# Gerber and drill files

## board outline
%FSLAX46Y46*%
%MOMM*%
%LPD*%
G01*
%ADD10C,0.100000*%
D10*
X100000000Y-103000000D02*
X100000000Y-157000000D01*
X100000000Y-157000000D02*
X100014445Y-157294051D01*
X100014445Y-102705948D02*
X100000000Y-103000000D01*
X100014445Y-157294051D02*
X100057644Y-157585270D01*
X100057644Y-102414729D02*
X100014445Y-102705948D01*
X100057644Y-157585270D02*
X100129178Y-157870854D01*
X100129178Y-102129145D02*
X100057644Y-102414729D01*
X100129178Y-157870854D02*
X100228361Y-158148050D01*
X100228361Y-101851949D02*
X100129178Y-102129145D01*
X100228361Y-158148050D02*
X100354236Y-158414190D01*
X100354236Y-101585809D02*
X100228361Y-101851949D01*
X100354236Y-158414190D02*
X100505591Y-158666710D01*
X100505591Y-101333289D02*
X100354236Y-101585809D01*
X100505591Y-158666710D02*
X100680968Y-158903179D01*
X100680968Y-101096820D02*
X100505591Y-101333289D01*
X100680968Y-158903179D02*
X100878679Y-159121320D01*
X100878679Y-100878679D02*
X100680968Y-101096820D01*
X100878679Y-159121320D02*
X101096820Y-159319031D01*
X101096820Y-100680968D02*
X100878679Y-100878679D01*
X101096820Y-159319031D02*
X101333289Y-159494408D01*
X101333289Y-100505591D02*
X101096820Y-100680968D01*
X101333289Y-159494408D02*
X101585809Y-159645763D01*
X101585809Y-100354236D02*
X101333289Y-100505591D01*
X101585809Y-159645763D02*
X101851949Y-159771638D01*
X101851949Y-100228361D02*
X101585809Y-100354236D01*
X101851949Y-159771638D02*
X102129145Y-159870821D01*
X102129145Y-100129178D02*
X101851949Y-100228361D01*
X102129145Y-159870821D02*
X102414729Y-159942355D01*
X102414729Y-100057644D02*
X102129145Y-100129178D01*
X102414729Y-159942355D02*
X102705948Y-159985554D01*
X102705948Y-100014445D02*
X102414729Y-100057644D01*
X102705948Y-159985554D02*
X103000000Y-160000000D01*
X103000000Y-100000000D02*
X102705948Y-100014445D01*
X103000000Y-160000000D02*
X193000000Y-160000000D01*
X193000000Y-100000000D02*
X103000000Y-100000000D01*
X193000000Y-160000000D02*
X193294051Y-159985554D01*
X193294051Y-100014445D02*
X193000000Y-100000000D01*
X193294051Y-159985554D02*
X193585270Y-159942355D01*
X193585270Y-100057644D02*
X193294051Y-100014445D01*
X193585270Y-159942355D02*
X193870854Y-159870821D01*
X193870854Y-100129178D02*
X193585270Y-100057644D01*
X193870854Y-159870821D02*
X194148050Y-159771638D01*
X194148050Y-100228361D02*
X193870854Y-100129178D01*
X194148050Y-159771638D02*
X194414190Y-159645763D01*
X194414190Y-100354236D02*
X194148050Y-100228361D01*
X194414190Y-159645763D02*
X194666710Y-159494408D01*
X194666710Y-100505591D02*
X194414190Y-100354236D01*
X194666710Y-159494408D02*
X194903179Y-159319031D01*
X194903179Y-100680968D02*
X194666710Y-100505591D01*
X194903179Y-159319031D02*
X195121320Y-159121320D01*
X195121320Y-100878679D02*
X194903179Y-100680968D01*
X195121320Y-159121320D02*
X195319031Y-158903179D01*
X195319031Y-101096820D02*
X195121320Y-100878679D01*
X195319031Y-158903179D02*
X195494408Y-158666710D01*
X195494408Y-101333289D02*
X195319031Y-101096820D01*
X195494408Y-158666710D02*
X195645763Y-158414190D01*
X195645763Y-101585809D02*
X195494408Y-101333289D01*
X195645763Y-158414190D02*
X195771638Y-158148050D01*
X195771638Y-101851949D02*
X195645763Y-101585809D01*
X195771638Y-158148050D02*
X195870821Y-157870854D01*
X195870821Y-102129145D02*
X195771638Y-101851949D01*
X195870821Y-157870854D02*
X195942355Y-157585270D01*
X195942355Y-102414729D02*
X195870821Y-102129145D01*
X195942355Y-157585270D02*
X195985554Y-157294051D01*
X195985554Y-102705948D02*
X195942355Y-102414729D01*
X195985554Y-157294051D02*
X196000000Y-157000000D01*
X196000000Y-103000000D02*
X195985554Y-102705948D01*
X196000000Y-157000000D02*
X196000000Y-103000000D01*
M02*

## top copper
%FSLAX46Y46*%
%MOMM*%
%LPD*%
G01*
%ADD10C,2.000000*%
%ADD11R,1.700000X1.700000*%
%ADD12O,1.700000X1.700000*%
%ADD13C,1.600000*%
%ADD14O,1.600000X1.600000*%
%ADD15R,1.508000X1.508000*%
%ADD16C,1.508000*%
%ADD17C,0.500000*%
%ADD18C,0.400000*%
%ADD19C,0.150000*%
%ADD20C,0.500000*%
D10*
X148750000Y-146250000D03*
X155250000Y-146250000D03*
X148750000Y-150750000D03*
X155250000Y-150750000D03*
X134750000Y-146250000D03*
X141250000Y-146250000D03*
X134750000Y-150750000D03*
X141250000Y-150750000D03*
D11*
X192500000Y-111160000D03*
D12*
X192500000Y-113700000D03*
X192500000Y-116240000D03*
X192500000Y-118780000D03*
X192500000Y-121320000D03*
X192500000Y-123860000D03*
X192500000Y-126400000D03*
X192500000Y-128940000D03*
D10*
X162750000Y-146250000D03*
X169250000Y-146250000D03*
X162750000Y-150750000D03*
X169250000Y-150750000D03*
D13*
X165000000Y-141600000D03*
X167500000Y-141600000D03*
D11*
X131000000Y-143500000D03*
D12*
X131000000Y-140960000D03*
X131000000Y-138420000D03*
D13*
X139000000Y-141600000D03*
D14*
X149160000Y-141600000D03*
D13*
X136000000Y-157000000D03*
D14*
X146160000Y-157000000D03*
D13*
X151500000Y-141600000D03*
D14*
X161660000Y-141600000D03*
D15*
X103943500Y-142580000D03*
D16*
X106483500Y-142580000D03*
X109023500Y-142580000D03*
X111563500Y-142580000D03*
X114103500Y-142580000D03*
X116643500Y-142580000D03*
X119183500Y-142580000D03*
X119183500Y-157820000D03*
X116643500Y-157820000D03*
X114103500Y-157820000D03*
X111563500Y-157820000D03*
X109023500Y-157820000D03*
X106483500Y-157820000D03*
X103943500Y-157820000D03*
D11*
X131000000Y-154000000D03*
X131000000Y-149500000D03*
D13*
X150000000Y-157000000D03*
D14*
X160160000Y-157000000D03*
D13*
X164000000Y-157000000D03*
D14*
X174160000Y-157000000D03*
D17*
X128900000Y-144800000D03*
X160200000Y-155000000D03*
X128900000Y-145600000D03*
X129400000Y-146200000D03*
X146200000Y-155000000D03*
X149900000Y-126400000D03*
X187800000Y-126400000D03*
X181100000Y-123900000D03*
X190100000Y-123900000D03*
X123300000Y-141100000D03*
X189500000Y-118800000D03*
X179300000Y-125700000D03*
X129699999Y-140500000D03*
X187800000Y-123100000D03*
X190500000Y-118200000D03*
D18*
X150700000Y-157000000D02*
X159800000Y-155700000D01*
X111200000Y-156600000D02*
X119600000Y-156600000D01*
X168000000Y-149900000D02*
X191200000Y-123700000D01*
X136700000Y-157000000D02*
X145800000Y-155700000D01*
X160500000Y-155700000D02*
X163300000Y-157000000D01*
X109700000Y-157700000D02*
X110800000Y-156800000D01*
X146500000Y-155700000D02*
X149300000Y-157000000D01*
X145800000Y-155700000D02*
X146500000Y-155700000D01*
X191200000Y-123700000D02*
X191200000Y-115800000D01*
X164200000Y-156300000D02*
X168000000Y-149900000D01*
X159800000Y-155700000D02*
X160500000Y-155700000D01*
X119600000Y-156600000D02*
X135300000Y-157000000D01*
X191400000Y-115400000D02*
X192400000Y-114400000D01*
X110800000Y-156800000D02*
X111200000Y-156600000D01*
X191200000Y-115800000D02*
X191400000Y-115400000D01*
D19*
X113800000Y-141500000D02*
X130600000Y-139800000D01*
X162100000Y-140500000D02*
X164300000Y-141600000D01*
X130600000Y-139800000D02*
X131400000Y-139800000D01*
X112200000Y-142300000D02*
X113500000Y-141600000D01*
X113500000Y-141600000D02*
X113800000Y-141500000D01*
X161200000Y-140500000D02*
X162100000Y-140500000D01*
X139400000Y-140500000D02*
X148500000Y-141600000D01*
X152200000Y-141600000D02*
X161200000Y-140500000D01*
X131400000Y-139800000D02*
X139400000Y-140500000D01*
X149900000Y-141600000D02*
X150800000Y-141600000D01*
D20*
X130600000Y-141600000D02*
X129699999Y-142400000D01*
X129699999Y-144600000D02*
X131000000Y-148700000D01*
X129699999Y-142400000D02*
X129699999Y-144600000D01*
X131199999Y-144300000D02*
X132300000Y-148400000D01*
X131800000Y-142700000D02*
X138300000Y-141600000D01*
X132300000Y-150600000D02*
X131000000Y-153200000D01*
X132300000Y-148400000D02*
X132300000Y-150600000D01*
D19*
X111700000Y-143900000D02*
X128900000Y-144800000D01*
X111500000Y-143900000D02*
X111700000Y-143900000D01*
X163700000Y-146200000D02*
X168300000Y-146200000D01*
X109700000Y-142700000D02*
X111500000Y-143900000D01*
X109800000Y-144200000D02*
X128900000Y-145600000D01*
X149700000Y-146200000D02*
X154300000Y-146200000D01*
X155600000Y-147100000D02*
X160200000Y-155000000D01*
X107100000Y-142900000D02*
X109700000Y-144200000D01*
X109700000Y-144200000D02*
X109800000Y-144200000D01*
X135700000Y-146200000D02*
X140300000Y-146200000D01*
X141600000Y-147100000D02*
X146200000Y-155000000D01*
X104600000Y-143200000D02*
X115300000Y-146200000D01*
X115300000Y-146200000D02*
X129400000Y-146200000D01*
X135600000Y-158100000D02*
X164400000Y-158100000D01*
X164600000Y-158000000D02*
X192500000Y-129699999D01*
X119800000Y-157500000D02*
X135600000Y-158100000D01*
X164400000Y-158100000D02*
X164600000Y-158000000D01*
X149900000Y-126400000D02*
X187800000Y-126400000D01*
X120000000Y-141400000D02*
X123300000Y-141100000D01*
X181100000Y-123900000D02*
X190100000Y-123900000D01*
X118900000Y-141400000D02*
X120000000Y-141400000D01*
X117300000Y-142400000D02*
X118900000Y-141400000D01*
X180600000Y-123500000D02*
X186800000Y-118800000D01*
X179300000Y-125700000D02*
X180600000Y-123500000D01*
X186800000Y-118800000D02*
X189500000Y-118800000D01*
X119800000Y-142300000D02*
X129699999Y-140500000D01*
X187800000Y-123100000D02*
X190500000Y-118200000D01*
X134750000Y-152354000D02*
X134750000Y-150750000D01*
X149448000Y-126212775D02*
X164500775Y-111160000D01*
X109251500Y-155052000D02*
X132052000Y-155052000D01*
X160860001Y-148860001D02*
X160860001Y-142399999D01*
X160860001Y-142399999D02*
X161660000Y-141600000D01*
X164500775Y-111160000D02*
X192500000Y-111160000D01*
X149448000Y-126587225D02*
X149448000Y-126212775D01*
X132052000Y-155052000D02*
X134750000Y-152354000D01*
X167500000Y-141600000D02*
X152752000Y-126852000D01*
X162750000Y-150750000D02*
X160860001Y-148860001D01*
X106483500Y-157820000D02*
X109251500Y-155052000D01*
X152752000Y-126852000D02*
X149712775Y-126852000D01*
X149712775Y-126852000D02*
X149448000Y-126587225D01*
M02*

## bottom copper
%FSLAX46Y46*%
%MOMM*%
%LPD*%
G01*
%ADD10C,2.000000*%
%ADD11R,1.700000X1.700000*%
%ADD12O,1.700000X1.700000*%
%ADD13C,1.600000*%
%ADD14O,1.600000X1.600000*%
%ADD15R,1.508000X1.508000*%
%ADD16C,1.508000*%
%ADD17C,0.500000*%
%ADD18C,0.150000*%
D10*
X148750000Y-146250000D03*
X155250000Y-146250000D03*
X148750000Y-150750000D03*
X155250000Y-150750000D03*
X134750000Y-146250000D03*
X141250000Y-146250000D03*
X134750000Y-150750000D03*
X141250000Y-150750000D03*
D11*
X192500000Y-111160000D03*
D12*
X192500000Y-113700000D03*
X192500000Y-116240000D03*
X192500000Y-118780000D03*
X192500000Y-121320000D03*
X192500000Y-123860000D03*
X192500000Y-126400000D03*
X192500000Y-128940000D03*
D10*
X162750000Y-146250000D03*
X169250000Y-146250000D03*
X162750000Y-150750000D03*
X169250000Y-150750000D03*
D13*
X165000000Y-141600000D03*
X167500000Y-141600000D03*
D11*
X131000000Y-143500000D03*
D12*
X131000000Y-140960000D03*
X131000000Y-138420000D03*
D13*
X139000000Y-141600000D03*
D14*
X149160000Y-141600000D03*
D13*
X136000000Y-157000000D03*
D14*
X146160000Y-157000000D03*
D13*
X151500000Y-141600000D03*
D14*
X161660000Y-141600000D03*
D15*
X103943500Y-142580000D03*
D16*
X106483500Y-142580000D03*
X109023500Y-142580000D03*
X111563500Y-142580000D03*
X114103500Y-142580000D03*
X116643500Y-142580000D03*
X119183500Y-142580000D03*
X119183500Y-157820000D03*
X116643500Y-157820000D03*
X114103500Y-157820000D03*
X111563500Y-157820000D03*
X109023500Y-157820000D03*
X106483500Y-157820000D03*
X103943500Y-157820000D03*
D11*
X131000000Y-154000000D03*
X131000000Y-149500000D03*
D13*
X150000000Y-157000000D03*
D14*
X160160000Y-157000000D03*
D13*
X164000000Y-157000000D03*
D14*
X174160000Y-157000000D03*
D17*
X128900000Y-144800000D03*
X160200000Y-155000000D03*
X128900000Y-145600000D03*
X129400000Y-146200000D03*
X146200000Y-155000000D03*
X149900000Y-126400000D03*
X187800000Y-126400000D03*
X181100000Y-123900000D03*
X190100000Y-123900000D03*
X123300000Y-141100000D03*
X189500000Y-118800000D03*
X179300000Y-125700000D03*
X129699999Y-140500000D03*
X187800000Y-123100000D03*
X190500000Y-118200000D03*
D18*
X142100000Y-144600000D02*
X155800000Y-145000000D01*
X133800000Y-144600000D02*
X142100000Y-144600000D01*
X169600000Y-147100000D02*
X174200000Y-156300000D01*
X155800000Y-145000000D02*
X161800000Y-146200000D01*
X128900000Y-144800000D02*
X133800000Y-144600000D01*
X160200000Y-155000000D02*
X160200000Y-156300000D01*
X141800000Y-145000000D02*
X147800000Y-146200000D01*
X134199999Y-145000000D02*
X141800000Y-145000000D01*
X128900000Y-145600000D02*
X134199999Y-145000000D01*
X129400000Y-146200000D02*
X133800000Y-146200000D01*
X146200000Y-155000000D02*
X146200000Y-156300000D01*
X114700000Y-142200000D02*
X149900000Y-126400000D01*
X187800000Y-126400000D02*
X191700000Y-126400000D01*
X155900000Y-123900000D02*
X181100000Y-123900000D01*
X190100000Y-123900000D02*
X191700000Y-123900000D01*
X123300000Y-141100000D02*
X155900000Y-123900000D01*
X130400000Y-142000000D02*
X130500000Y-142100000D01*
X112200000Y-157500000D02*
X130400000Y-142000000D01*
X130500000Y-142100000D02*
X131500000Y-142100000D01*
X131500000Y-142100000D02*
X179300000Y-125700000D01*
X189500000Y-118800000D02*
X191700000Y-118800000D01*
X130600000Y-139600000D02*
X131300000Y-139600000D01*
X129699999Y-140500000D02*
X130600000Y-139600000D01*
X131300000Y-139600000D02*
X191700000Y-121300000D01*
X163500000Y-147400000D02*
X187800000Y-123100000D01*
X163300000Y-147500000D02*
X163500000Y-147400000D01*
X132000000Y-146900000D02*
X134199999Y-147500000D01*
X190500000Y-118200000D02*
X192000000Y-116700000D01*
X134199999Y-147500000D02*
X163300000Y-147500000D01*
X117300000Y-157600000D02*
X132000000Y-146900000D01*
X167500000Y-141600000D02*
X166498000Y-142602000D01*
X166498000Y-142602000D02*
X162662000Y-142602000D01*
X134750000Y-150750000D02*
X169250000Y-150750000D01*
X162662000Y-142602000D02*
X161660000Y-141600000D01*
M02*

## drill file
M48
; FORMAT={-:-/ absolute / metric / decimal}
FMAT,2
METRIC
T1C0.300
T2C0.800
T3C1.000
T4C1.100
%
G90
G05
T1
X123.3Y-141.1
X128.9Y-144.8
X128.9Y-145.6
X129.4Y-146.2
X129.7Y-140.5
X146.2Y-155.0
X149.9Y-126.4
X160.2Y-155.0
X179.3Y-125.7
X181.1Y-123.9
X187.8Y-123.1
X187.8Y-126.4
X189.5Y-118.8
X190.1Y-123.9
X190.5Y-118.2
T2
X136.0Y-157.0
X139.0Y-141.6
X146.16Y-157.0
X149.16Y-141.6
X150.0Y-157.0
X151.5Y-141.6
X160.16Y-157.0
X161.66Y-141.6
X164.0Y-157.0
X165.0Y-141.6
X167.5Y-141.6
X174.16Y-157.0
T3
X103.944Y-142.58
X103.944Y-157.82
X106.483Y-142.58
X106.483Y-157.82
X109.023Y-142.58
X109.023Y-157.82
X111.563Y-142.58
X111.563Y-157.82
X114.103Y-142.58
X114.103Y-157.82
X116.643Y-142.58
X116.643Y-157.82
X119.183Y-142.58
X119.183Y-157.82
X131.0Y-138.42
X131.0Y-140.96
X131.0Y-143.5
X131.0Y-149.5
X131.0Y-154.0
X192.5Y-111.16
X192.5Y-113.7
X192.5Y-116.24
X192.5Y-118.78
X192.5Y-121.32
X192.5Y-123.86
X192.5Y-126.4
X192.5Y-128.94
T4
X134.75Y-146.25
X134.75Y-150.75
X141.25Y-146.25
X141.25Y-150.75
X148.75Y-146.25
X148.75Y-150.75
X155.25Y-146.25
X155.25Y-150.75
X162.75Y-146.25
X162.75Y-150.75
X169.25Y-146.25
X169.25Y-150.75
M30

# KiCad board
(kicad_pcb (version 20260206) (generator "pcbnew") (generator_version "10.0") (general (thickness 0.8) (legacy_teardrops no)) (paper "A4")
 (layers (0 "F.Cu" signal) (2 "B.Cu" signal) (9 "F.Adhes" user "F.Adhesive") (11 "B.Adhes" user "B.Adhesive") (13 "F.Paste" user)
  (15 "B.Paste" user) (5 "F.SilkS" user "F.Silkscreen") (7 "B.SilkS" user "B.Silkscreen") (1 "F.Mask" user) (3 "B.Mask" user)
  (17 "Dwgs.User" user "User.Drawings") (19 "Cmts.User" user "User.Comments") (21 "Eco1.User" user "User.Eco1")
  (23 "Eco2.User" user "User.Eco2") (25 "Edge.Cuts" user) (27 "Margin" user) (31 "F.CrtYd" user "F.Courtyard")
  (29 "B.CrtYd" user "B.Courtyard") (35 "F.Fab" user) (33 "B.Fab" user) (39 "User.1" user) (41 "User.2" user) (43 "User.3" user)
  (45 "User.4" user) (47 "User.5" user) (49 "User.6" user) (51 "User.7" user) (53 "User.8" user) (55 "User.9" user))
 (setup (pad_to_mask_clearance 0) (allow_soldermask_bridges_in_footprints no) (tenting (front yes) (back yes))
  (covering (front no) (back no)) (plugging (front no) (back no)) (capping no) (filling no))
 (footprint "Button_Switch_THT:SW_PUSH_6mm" (layer "F.Cu") (at 148.75 146.25)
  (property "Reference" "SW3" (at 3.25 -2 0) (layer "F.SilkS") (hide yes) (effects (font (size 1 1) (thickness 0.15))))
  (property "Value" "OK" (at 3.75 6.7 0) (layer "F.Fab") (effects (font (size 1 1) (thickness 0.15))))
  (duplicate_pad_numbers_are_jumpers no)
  (pad "1" thru_hole circle (at 0 0 90) (size 2 2) (drill 1.1) (layers "*.Cu" "*.Mask") (remove_unused_layers no) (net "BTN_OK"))
  (pad "1" thru_hole circle (at 6.5 0 90) (size 2 2) (drill 1.1) (layers "*.Cu" "*.Mask") (remove_unused_layers no) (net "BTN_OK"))
  (pad "2" thru_hole circle (at 0 4.5 90) (size 2 2) (drill 1.1) (layers "*.Cu" "*.Mask") (remove_unused_layers no) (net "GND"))
  (pad "2" thru_hole circle (at 6.5 4.5 90) (size 2 2) (drill 1.1) (layers "*.Cu" "*.Mask") (remove_unused_layers no) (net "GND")))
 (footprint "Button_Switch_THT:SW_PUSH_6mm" (layer "F.Cu") (at 134.75 146.25)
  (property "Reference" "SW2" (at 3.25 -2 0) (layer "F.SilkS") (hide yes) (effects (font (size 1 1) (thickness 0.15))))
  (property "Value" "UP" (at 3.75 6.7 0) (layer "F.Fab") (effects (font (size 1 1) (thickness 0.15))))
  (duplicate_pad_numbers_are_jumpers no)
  (pad "1" thru_hole circle (at 0 0 90) (size 2 2) (drill 1.1) (layers "*.Cu" "*.Mask") (remove_unused_layers no) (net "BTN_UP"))
  (pad "1" thru_hole circle (at 6.5 0 90) (size 2 2) (drill 1.1) (layers "*.Cu" "*.Mask") (remove_unused_layers no) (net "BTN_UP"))
  (pad "2" thru_hole circle (at 0 4.5 90) (size 2 2) (drill 1.1) (layers "*.Cu" "*.Mask") (remove_unused_layers no) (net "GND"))
  (pad "2" thru_hole circle (at 6.5 4.5 90) (size 2 2) (drill 1.1) (layers "*.Cu" "*.Mask") (remove_unused_layers no) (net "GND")))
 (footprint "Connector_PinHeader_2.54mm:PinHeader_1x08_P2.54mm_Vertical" (layer "F.Cu") (at 192.5 111.16)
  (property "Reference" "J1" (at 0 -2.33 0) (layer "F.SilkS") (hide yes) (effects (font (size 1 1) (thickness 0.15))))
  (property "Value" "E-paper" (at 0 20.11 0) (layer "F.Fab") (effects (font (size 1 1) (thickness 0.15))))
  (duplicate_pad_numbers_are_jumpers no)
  (pad "1" thru_hole rect (at 0 0) (size 1.7 1.7) (drill 1) (layers "*.Cu" "*.Mask") (remove_unused_layers no) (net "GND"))
  (pad "2" thru_hole oval (at 0 2.54) (size 1.7 1.7) (drill 1) (layers "*.Cu" "*.Mask") (remove_unused_layers no) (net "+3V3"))
  (pad "3" thru_hole oval (at 0 5.08) (size 1.7 1.7) (drill 1) (layers "*.Cu" "*.Mask") (remove_unused_layers no) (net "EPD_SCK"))
  (pad "4" thru_hole oval (at 0 7.62) (size 1.7 1.7) (drill 1) (layers "*.Cu" "*.Mask") (remove_unused_layers no) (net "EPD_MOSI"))
  (pad "5" thru_hole oval (at 0 10.16) (size 1.7 1.7) (drill 1) (layers "*.Cu" "*.Mask") (remove_unused_layers no) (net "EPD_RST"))
  (pad "6" thru_hole oval (at 0 12.7) (size 1.7 1.7) (drill 1) (layers "*.Cu" "*.Mask") (remove_unused_layers no) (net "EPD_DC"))
  (pad "7" thru_hole oval (at 0 15.24) (size 1.7 1.7) (drill 1) (layers "*.Cu" "*.Mask") (remove_unused_layers no) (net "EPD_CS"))
  (pad "8" thru_hole oval (at 0 17.78) (size 1.7 1.7) (drill 1) (layers "*.Cu" "*.Mask") (remove_unused_layers no) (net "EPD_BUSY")))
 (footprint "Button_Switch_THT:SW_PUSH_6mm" (layer "F.Cu") (at 162.75 146.25)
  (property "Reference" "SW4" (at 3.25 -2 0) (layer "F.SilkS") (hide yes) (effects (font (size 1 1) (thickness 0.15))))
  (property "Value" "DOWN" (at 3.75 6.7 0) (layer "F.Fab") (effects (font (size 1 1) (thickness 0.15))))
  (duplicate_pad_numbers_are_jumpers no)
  (pad "1" thru_hole circle (at 0 0 90) (size 2 2) (drill 1.1) (layers "*.Cu" "*.Mask") (remove_unused_layers no) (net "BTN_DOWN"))
  (pad "1" thru_hole circle (at 6.5 0 90) (size 2 2) (drill 1.1) (layers "*.Cu" "*.Mask") (remove_unused_layers no) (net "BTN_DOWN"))
  (pad "2" thru_hole circle (at 0 4.5 90) (size 2 2) (drill 1.1) (layers "*.Cu" "*.Mask") (remove_unused_layers no) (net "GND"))
  (pad "2" thru_hole circle (at 6.5 4.5 90) (size 2 2) (drill 1.1) (layers "*.Cu" "*.Mask") (remove_unused_layers no) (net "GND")))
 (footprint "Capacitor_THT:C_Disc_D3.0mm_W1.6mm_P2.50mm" (layer "B.Cu") (at 165 141.6)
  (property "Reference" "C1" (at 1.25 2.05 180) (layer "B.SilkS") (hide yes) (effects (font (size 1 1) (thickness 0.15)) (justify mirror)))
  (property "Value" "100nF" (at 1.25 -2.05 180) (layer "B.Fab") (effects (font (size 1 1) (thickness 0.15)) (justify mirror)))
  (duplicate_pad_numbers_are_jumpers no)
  (pad "1" thru_hole circle (at 0 0) (size 1.6 1.6) (drill 0.8) (layers "*.Cu" "*.Mask") (remove_unused_layers no) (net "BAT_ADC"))
  (pad "2" thru_hole circle (at 2.5 0) (size 1.6 1.6) (drill 0.8) (layers "*.Cu" "*.Mask") (remove_unused_layers no) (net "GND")))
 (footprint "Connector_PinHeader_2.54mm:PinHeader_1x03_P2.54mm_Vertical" (layer "B.Cu") (at 131 143.5)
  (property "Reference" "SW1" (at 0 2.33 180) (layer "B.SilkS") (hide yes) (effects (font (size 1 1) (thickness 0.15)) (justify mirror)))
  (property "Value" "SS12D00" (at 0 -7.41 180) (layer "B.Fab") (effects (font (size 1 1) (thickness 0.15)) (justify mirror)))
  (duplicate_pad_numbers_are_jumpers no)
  (pad "1" thru_hole rect (at 0 0) (size 1.7 1.7) (drill 1) (layers "*.Cu" "*.Mask") (remove_unused_layers no) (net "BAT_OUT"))
  (pad "2" thru_hole oval (at 0 -2.54) (size 1.7 1.7) (drill 1) (layers "*.Cu" "*.Mask") (remove_unused_layers no) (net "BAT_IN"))
  (pad "3" thru_hole oval (at 0 -5.08) (size 1.7 1.7) (drill 1) (layers "*.Cu" "*.Mask") (remove_unused_layers no)))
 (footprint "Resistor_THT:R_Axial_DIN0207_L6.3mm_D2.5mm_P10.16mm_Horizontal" (layer "B.Cu") (at 139 141.6)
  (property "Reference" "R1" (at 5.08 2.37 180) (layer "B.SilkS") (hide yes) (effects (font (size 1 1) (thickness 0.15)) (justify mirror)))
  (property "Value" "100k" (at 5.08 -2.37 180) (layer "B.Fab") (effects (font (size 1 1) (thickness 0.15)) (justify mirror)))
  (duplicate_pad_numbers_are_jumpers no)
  (pad "1" thru_hole circle (at 0 0) (size 1.6 1.6) (drill 0.8) (layers "*.Cu" "*.Mask") (remove_unused_layers no) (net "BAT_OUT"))
  (pad "2" thru_hole oval (at 10.16 0) (size 1.6 1.6) (drill 0.8) (layers "*.Cu" "*.Mask") (remove_unused_layers no) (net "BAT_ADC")))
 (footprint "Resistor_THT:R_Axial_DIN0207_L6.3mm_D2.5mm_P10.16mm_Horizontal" (layer "B.Cu") (at 136 157)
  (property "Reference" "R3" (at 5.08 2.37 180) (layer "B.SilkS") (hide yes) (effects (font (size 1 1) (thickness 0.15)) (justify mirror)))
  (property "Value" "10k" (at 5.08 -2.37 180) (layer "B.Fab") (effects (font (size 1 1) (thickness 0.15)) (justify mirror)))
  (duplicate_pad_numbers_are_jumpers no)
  (pad "1" thru_hole circle (at 0 0) (size 1.6 1.6) (drill 0.8) (layers "*.Cu" "*.Mask") (remove_unused_layers no) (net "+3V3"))
  (pad "2" thru_hole oval (at 10.16 0) (size 1.6 1.6) (drill 0.8) (layers "*.Cu" "*.Mask") (remove_unused_layers no) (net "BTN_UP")))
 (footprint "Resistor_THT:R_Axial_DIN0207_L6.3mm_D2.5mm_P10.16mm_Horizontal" (layer "B.Cu") (at 151.5 141.6)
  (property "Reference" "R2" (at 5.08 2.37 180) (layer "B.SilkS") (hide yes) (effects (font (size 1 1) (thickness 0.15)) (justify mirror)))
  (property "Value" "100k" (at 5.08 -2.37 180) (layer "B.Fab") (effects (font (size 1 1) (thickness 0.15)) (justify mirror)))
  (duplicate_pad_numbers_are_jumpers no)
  (pad "1" thru_hole circle (at 0 0) (size 1.6 1.6) (drill 0.8) (layers "*.Cu" "*.Mask") (remove_unused_layers no) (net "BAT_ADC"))
  (pad "2" thru_hole oval (at 10.16 0) (size 1.6 1.6) (drill 0.8) (layers "*.Cu" "*.Mask") (remove_unused_layers no) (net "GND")))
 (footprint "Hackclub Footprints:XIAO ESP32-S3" (layer "B.Cu") (at 111.5 150.2 -90)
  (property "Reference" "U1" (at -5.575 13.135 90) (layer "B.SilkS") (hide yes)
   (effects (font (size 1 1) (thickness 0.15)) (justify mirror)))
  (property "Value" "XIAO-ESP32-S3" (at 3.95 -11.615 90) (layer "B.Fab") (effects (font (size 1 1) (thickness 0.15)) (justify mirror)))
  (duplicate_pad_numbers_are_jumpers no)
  (pad "1" thru_hole rect (at -7.62 7.5565 270) (size 1.508 1.508) (drill 1) (layers "*.Cu" "*.Mask") (remove_unused_layers no)
   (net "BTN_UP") (solder_mask_margin 0.102))
  (pad "2" thru_hole circle (at -7.62 5.0165 270) (size 1.508 1.508) (drill 1) (layers "*.Cu" "*.Mask") (remove_unused_layers no)
   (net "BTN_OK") (solder_mask_margin 0.102))
  (pad "3" thru_hole circle (at -7.62 2.4765 270) (size 1.508 1.508) (drill 1) (layers "*.Cu" "*.Mask") (remove_unused_layers no)
   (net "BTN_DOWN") (solder_mask_margin 0.102))
  (pad "4" thru_hole circle (at -7.62 -0.0635 270) (size 1.508 1.508) (drill 1) (layers "*.Cu" "*.Mask") (remove_unused_layers no)
   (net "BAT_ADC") (solder_mask_margin 0.102))
  (pad "5" thru_hole circle (at -7.62 -2.6035 270) (size 1.508 1.508) (drill 1) (layers "*.Cu" "*.Mask") (remove_unused_layers no)
   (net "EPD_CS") (solder_mask_margin 0.102))
  (pad "6" thru_hole circle (at -7.62 -5.1435 270) (size 1.508 1.508) (drill 1) (layers "*.Cu" "*.Mask") (remove_unused_layers no)
   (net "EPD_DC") (solder_mask_margin 0.102))
  (pad "7" thru_hole circle (at -7.62 -7.6835 270) (size 1.508 1.508) (drill 1) (layers "*.Cu" "*.Mask") (remove_unused_layers no)
   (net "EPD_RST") (solder_mask_margin 0.102))
  (pad "8" thru_hole circle (at 7.62 -7.6835 270) (size 1.508 1.508) (drill 1) (layers "*.Cu" "*.Mask") (remove_unused_layers no)
   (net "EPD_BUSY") (solder_mask_margin 0.102))
  (pad "9" thru_hole circle (at 7.62 -5.1435 270) (size 1.508 1.508) (drill 1) (layers "*.Cu" "*.Mask") (remove_unused_layers no)
   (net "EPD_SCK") (solder_mask_margin 0.102))
  (pad "10" thru_hole circle (at 7.62 -2.6035 270) (size 1.508 1.508) (drill 1) (layers "*.Cu" "*.Mask") (remove_unused_layers no)
   (solder_mask_margin 0.102))
  (pad "11" thru_hole circle (at 7.62 -0.0635 270) (size 1.508 1.508) (drill 1) (layers "*.Cu" "*.Mask") (remove_unused_layers no)
   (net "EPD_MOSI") (solder_mask_margin 0.102))
  (pad "12" thru_hole circle (at 7.62 2.4765 270) (size 1.508 1.508) (drill 1) (layers "*.Cu" "*.Mask") (remove_unused_layers no)
   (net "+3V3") (solder_mask_margin 0.102))
  (pad "13" thru_hole circle (at 7.62 5.0165 270) (size 1.508 1.508) (drill 1) (layers "*.Cu" "*.Mask") (remove_unused_layers no)
   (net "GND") (solder_mask_margin 0.102))
  (pad "14" thru_hole circle (at 7.62 7.5565 270) (size 1.508 1.508) (drill 1) (layers "*.Cu" "*.Mask") (remove_unused_layers no)
   (solder_mask_margin 0.102)))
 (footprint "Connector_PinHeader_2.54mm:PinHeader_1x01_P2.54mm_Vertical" (layer "B.Cu") (at 131 154)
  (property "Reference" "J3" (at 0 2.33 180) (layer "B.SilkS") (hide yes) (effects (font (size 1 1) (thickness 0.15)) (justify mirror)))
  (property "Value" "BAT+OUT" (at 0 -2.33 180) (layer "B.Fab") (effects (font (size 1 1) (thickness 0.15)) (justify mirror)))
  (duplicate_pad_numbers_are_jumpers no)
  (pad "1" thru_hole rect (at 0 0) (size 1.7 1.7) (drill 1) (layers "*.Cu" "*.Mask") (remove_unused_layers no) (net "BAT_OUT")))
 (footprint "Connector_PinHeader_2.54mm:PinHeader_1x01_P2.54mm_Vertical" (layer "B.Cu") (at 131 149.5)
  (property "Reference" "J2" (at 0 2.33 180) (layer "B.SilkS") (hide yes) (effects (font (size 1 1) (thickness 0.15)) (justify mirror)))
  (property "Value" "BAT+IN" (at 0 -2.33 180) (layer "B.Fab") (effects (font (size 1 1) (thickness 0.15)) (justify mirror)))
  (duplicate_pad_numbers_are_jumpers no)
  (pad "1" thru_hole rect (at 0 0) (size 1.7 1.7) (drill 1) (layers "*.Cu" "*.Mask") (remove_unused_layers no) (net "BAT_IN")))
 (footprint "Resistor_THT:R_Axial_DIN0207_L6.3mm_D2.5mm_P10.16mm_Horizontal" (layer "B.Cu") (at 150 157)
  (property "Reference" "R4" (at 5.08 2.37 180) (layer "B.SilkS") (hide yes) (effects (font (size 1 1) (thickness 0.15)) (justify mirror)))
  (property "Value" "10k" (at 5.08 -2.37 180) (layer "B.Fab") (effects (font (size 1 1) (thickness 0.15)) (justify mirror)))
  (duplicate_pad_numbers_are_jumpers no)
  (pad "1" thru_hole circle (at 0 0) (size 1.6 1.6) (drill 0.8) (layers "*.Cu" "*.Mask") (remove_unused_layers no) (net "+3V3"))
  (pad "2" thru_hole oval (at 10.16 0) (size 1.6 1.6) (drill 0.8) (layers "*.Cu" "*.Mask") (remove_unused_layers no) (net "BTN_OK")))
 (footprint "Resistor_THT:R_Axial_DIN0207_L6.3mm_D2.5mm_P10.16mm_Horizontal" (layer "B.Cu") (at 164 157)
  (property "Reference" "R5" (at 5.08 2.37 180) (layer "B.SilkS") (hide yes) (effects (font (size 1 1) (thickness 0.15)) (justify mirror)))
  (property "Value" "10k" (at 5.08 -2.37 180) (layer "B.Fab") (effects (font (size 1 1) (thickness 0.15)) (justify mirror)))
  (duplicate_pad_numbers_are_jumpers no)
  (pad "1" thru_hole circle (at 0 0) (size 1.6 1.6) (drill 0.8) (layers "*.Cu" "*.Mask") (remove_unused_layers no) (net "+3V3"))
  (pad "2" thru_hole oval (at 10.16 0) (size 1.6 1.6) (drill 0.8) (layers "*.Cu" "*.Mask") (remove_unused_layers no) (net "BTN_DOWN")))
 (gr_line (start 100 103) (end 100 157) (stroke (width 0.1) (type default)) (layer "Edge.Cuts"))
 (gr_line (start 100 157) (end 100.014445 157.294051) (stroke (width 0.1) (type default)) (layer "Edge.Cuts"))
 (gr_line (start 100.014445 102.705948) (end 100 103) (stroke (width 0.1) (type default)) (layer "Edge.Cuts"))
 (gr_line (start 100.014445 157.294051) (end 100.057644 157.58527) (stroke (width 0.1) (type default)) (layer "Edge.Cuts"))
 (gr_line (start 100.057644 102.414729) (end 100.014445 102.705948) (stroke (width 0.1) (type default)) (layer "Edge.Cuts"))
 (gr_line (start 100.057644 157.58527) (end 100.129178 157.870854) (stroke (width 0.1) (type default)) (layer "Edge.Cuts"))
 (gr_line (start 100.129178 102.129145) (end 100.057644 102.414729) (stroke (width 0.1) (type default)) (layer "Edge.Cuts"))
 (gr_line (start 100.129178 157.870854) (end 100.228361 158.14805) (stroke (width 0.1) (type default)) (layer "Edge.Cuts"))
 (gr_line (start 100.228361 101.851949) (end 100.129178 102.129145) (stroke (width 0.1) (type default)) (layer "Edge.Cuts"))
 (gr_line (start 100.228361 158.14805) (end 100.354236 158.41419) (stroke (width 0.1) (type default)) (layer "Edge.Cuts"))
 (gr_line (start 100.354236 101.585809) (end 100.228361 101.851949) (stroke (width 0.1) (type default)) (layer "Edge.Cuts"))
 (gr_line (start 100.354236 158.41419) (end 100.505591 158.66671) (stroke (width 0.1) (type default)) (layer "Edge.Cuts"))
 (gr_line (start 100.505591 101.333289) (end 100.354236 101.585809) (stroke (width 0.1) (type default)) (layer "Edge.Cuts"))
 (gr_line (start 100.505591 158.66671) (end 100.680968 158.903179) (stroke (width 0.1) (type default)) (layer "Edge.Cuts"))
 (gr_line (start 100.680968 101.09682) (end 100.505591 101.333289) (stroke (width 0.1) (type default)) (layer "Edge.Cuts"))
 (gr_line (start 100.680968 158.903179) (end 100.878679 159.12132) (stroke (width 0.1) (type default)) (layer "Edge.Cuts"))
 (gr_line (start 100.878679 100.878679) (end 100.680968 101.09682) (stroke (width 0.1) (type default)) (layer "Edge.Cuts"))
 (gr_line (start 100.878679 159.12132) (end 101.09682 159.319031) (stroke (width 0.1) (type default)) (layer "Edge.Cuts"))
 (gr_line (start 101.09682 100.680968) (end 100.878679 100.878679) (stroke (width 0.1) (type default)) (layer "Edge.Cuts"))
 (gr_line (start 101.09682 159.319031) (end 101.333289 159.494408) (stroke (width 0.1) (type default)) (layer "Edge.Cuts"))
 (gr_line (start 101.333289 100.505591) (end 101.09682 100.680968) (stroke (width 0.1) (type default)) (layer "Edge.Cuts"))
 (gr_line (start 101.333289 159.494408) (end 101.585809 159.645763) (stroke (width 0.1) (type default)) (layer "Edge.Cuts"))
 (gr_line (start 101.585809 100.354236) (end 101.333289 100.505591) (stroke (width 0.1) (type default)) (layer "Edge.Cuts"))
 (gr_line (start 101.585809 159.645763) (end 101.851949 159.771638) (stroke (width 0.1) (type default)) (layer "Edge.Cuts"))
 (gr_line (start 101.851949 100.228361) (end 101.585809 100.354236) (stroke (width 0.1) (type default)) (layer "Edge.Cuts"))
 (gr_line (start 101.851949 159.771638) (end 102.129145 159.870821) (stroke (width 0.1) (type default)) (layer "Edge.Cuts"))
 (gr_line (start 102.129145 100.129178) (end 101.851949 100.228361) (stroke (width 0.1) (type default)) (layer "Edge.Cuts"))
 (gr_line (start 102.129145 159.870821) (end 102.414729 159.942355) (stroke (width 0.1) (type default)) (layer "Edge.Cuts"))
 (gr_line (start 102.414729 100.057644) (end 102.129145 100.129178) (stroke (width 0.1) (type default)) (layer "Edge.Cuts"))
 (gr_line (start 102.414729 159.942355) (end 102.705948 159.985554) (stroke (width 0.1) (type default)) (layer "Edge.Cuts"))
 (gr_line (start 102.705948 100.014445) (end 102.414729 100.057644) (stroke (width 0.1) (type default)) (layer "Edge.Cuts"))
 (gr_line (start 102.705948 159.985554) (end 103 160) (stroke (width 0.1) (type default)) (layer "Edge.Cuts"))
 (gr_line (start 103 100) (end 102.705948 100.014445) (stroke (width 0.1) (type default)) (layer "Edge.Cuts"))
 (gr_line (start 103 160) (end 193 160) (stroke (width 0.1) (type default)) (layer "Edge.Cuts"))
 (gr_line (start 193 100) (end 103 100) (stroke (width 0.1) (type default)) (layer "Edge.Cuts"))
 (gr_line (start 193 160) (end 193.294051 159.985554) (stroke (width 0.1) (type default)) (layer "Edge.Cuts"))
 (gr_line (start 193.294051 100.014445) (end 193 100) (stroke (width 0.1) (type default)) (layer "Edge.Cuts"))
 (gr_line (start 193.294051 159.985554) (end 193.58527 159.942355) (stroke (width 0.1) (type default)) (layer "Edge.Cuts"))
 (gr_line (start 193.58527 100.057644) (end 193.294051 100.014445) (stroke (width 0.1) (type default)) (layer "Edge.Cuts"))
 (gr_line (start 193.58527 159.942355) (end 193.870854 159.870821) (stroke (width 0.1) (type default)) (layer "Edge.Cuts"))
 (gr_line (start 193.870854 100.129178) (end 193.58527 100.057644) (stroke (width 0.1) (type default)) (layer "Edge.Cuts"))
 (gr_line (start 193.870854 159.870821) (end 194.14805 159.771638) (stroke (width 0.1) (type default)) (layer "Edge.Cuts"))
 (gr_line (start 194.14805 100.228361) (end 193.870854 100.129178) (stroke (width 0.1) (type default)) (layer "Edge.Cuts"))
 (gr_line (start 194.14805 159.771638) (end 194.41419 159.645763) (stroke (width 0.1) (type default)) (layer "Edge.Cuts"))
 (gr_line (start 194.41419 100.354236) (end 194.14805 100.228361) (stroke (width 0.1) (type default)) (layer "Edge.Cuts"))
 (gr_line (start 194.41419 159.645763) (end 194.66671 159.494408) (stroke (width 0.1) (type default)) (layer "Edge.Cuts"))
 (gr_line (start 194.66671 100.505591) (end 194.41419 100.354236) (stroke (width 0.1) (type default)) (layer "Edge.Cuts"))
 (gr_line (start 194.66671 159.494408) (end 194.903179 159.319031) (stroke (width 0.1) (type default)) (layer "Edge.Cuts"))
 (gr_line (start 194.903179 100.680968) (end 194.66671 100.505591) (stroke (width 0.1) (type default)) (layer "Edge.Cuts"))
 (gr_line (start 194.903179 159.319031) (end 195.12132 159.12132) (stroke (width 0.1) (type default)) (layer "Edge.Cuts"))
 (gr_line (start 195.12132 100.878679) (end 194.903179 100.680968) (stroke (width 0.1) (type default)) (layer "Edge.Cuts"))
 (gr_line (start 195.12132 159.12132) (end 195.319031 158.903179) (stroke (width 0.1) (type default)) (layer "Edge.Cuts"))
 (gr_line (start 195.319031 101.09682) (end 195.12132 100.878679) (stroke (width 0.1) (type default)) (layer "Edge.Cuts"))
 (gr_line (start 195.319031 158.903179) (end 195.494408 158.66671) (stroke (width 0.1) (type default)) (layer "Edge.Cuts"))
 (gr_line (start 195.494408 101.333289) (end 195.319031 101.09682) (stroke (width 0.1) (type default)) (layer "Edge.Cuts"))
 (gr_line (start 195.494408 158.66671) (end 195.645763 158.41419) (stroke (width 0.1) (type default)) (layer "Edge.Cuts"))
 (gr_line (start 195.645763 101.585809) (end 195.494408 101.333289) (stroke (width 0.1) (type default)) (layer "Edge.Cuts"))
 (gr_line (start 195.645763 158.41419) (end 195.771638 158.14805) (stroke (width 0.1) (type default)) (layer "Edge.Cuts"))
 (gr_line (start 195.771638 101.851949) (end 195.645763 101.585809) (stroke (width 0.1) (type default)) (layer "Edge.Cuts"))
 (gr_line (start 195.771638 158.14805) (end 195.870821 157.870854) (stroke (width 0.1) (type default)) (layer "Edge.Cuts"))
 (gr_line (start 195.870821 102.129145) (end 195.771638 101.851949) (stroke (width 0.1) (type default)) (layer "Edge.Cuts"))
 (gr_line (start 195.870821 157.870854) (end 195.942355 157.58527) (stroke (width 0.1) (type default)) (layer "Edge.Cuts"))
 (gr_line (start 195.942355 102.414729) (end 195.870821 102.129145) (stroke (width 0.1) (type default)) (layer "Edge.Cuts"))
 (gr_line (start 195.942355 157.58527) (end 195.985554 157.294051) (stroke (width 0.1) (type default)) (layer "Edge.Cuts"))
 (gr_line (start 195.985554 102.705948) (end 195.942355 102.414729) (stroke (width 0.1) (type default)) (layer "Edge.Cuts"))
 (gr_line (start 195.985554 157.294051) (end 196 157) (stroke (width 0.1) (type default)) (layer "Edge.Cuts"))
 (gr_line (start 196 103) (end 195.985554 102.705948) (stroke (width 0.1) (type default)) (layer "Edge.Cuts"))
 (gr_line (start 196 157) (end 196 103) (stroke (width 0.1) (type default)) (layer "Edge.Cuts"))
 (segment (start 150.7 157) (end 159.8 155.7) (width 0.4) (layer "F.Cu") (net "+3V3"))
 (segment (start 111.2 156.6) (end 119.6 156.6) (width 0.4) (layer "F.Cu") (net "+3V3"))
 (segment (start 168 149.9) (end 191.2 123.7) (width 0.4) (layer "F.Cu") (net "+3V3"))
 (segment (start 136.7 157) (end 145.8 155.7) (width 0.4) (layer "F.Cu") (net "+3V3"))
 (segment (start 160.5 155.7) (end 163.3 157) (width 0.4) (layer "F.Cu") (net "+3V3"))
 (segment (start 109.7 157.7) (end 110.8 156.8) (width 0.4) (layer "F.Cu") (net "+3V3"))
 (segment (start 146.5 155.7) (end 149.3 157) (width 0.4) (layer "F.Cu") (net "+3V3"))
 (segment (start 145.8 155.7) (end 146.5 155.7) (width 0.4) (layer "F.Cu") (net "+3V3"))
 (segment (start 191.2 123.7) (end 191.2 115.8) (width 0.4) (layer "F.Cu") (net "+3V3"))
 (segment (start 164.2 156.3) (end 168 149.9) (width 0.4) (layer "F.Cu") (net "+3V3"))
 (segment (start 159.8 155.7) (end 160.5 155.7) (width 0.4) (layer "F.Cu") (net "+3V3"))
 (segment (start 119.6 156.6) (end 135.3 157) (width 0.4) (layer "F.Cu") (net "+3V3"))
 (segment (start 191.4 115.4) (end 192.4 114.4) (width 0.4) (layer "F.Cu") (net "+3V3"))
 (segment (start 110.8 156.8) (end 111.2 156.6) (width 0.4) (layer "F.Cu") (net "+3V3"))
 (segment (start 191.2 115.8) (end 191.4 115.4) (width 0.4) (layer "F.Cu") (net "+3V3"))
 (segment (start 113.8 141.5) (end 130.6 139.8) (width 0.15) (layer "F.Cu") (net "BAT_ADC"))
 (segment (start 162.1 140.5) (end 164.3 141.6) (width 0.15) (layer "F.Cu") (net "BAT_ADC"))
 (segment (start 130.6 139.8) (end 131.4 139.8) (width 0.15) (layer "F.Cu") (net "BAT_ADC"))
 (segment (start 112.2 142.3) (end 113.5 141.6) (width 0.15) (layer "F.Cu") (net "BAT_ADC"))
 (segment (start 113.5 141.6) (end 113.8 141.5) (width 0.15) (layer "F.Cu") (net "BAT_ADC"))
 (segment (start 161.2 140.5) (end 162.1 140.5) (width 0.15) (layer "F.Cu") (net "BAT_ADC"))
 (segment (start 139.4 140.5) (end 148.5 141.6) (width 0.15) (layer "F.Cu") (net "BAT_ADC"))
 (segment (start 152.2 141.6) (end 161.2 140.5) (width 0.15) (layer "F.Cu") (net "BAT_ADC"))
 (segment (start 131.4 139.8) (end 139.4 140.5) (width 0.15) (layer "F.Cu") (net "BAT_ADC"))
 (segment (start 149.9 141.6) (end 150.8 141.6) (width 0.15) (layer "F.Cu") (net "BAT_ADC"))
 (segment (start 130.6 141.6) (end 129.699999 142.4) (width 0.5) (layer "F.Cu") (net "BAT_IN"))
 (segment (start 129.699999 144.6) (end 131 148.7) (width 0.5) (layer "F.Cu") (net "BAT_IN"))
 (segment (start 129.699999 142.4) (end 129.699999 144.6) (width 0.5) (layer "F.Cu") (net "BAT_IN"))
 (segment (start 131.199999 144.3) (end 132.3 148.4) (width 0.5) (layer "F.Cu") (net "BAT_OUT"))
 (segment (start 131.8 142.7) (end 138.3 141.6) (width 0.5) (layer "F.Cu") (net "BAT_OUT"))
 (segment (start 132.3 150.6) (end 131 153.2) (width 0.5) (layer "F.Cu") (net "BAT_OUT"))
 (segment (start 132.3 148.4) (end 132.3 150.6) (width 0.5) (layer "F.Cu") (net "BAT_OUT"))
 (segment (start 111.7 143.9) (end 128.9 144.8) (width 0.15) (layer "F.Cu") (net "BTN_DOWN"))
 (segment (start 111.5 143.9) (end 111.7 143.9) (width 0.15) (layer "F.Cu") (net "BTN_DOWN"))
 (segment (start 163.7 146.2) (end 168.3 146.2) (width 0.15) (layer "F.Cu") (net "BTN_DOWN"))
 (segment (start 109.7 142.7) (end 111.5 143.9) (width 0.15) (layer "F.Cu") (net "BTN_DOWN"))
 (via (at 128.9 144.8) (size 0.5) (drill 0.3) (layers "F.Cu" "B.Cu") (capping no) (covering (front no) (back no))
  (plugging (front no) (back no)) (filling no) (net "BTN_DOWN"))
 (segment (start 142.1 144.6) (end 155.8 145) (width 0.15) (layer "B.Cu") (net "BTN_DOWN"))
 (segment (start 133.8 144.6) (end 142.1 144.6) (width 0.15) (layer "B.Cu") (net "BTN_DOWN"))
 (segment (start 169.6 147.1) (end 174.2 156.3) (width 0.15) (layer "B.Cu") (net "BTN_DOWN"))
 (segment (start 155.8 145) (end 161.8 146.2) (width 0.15) (layer "B.Cu") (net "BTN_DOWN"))
 (segment (start 128.9 144.8) (end 133.8 144.6) (width 0.15) (layer "B.Cu") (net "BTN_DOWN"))
 (segment (start 109.8 144.2) (end 128.9 145.6) (width 0.15) (layer "F.Cu") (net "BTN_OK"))
 (segment (start 149.7 146.2) (end 154.3 146.2) (width 0.15) (layer "F.Cu") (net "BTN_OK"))
 (segment (start 155.6 147.1) (end 160.2 155) (width 0.15) (layer "F.Cu") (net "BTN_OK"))
 (segment (start 107.1 142.9) (end 109.7 144.2) (width 0.15) (layer "F.Cu") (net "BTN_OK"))
 (segment (start 109.7 144.2) (end 109.8 144.2) (width 0.15) (layer "F.Cu") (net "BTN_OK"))
 (via (at 160.2 155) (size 0.5) (drill 0.3) (layers "F.Cu" "B.Cu") (capping no) (covering (front no) (back no))
  (plugging (front no) (back no)) (filling no) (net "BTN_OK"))
 (via (at 128.9 145.6) (size 0.5) (drill 0.3) (layers "F.Cu" "B.Cu") (capping no) (covering (front no) (back no))
  (plugging (front no) (back no)) (filling no) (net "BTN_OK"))
 (segment (start 160.2 155) (end 160.2 156.3) (width 0.15) (layer "B.Cu") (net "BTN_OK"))
 (segment (start 141.8 145) (end 147.8 146.2) (width 0.15) (layer "B.Cu") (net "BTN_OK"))
 (segment (start 134.199999 145) (end 141.8 145) (width 0.15) (layer "B.Cu") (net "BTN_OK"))
 (segment (start 128.9 145.6) (end 134.199999 145) (width 0.15) (layer "B.Cu") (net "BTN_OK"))
 (segment (start 135.7 146.2) (end 140.3 146.2) (width 0.15) (layer "F.Cu") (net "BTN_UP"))
 (segment (start 141.6 147.1) (end 146.2 155) (width 0.15) (layer "F.Cu") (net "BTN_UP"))
 (segment (start 104.6 143.2) (end 115.3 146.2) (width 0.15) (layer "F.Cu") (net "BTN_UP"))
 (segment (start 115.3 146.2) (end 129.4 146.2) (width 0.15) (layer "F.Cu") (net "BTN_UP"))
 (via (at 129.4 146.2) (size 0.5) (drill 0.3) (layers "F.Cu" "B.Cu") (capping no) (covering (front no) (back no))
  (plugging (front no) (back no)) (filling no) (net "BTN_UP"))
 (via (at 146.2 155) (size 0.5) (drill 0.3) (layers "F.Cu" "B.Cu") (capping no) (covering (front no) (back no))
  (plugging (front no) (back no)) (filling no) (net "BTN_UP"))
 (segment (start 129.4 146.2) (end 133.8 146.2) (width 0.15) (layer "B.Cu") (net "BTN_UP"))
 (segment (start 146.2 155) (end 146.2 156.3) (width 0.15) (layer "B.Cu") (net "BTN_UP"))
 (segment (start 135.6 158.1) (end 164.4 158.1) (width 0.15) (layer "F.Cu") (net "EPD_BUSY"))
 (segment (start 164.6 158) (end 192.5 129.699999) (width 0.15) (layer "F.Cu") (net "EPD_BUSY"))
 (segment (start 119.8 157.5) (end 135.6 158.1) (width 0.15) (layer "F.Cu") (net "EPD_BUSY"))
 (segment (start 164.4 158.1) (end 164.6 158) (width 0.15) (layer "F.Cu") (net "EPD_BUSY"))
 (segment (start 149.9 126.4) (end 187.8 126.4) (width 0.15) (layer "F.Cu") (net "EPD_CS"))
 (via (at 149.9 126.4) (size 0.5) (drill 0.3) (layers "F.Cu" "B.Cu") (capping no) (covering (front no) (back no))
  (plugging (front no) (back no)) (filling no) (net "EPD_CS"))
 (via (at 187.8 126.4) (size 0.5) (drill 0.3) (layers "F.Cu" "B.Cu") (capping no) (covering (front no) (back no))
  (plugging (front no) (back no)) (filling no) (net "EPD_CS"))
 (segment (start 114.7 142.2) (end 149.9 126.4) (width 0.15) (layer "B.Cu") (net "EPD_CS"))
 (segment (start 187.8 126.4) (end 191.7 126.4) (width 0.15) (layer "B.Cu") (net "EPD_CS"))
 (segment (start 120 141.4) (end 123.3 141.1) (width 0.15) (layer "F.Cu") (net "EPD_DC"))
 (segment (start 181.1 123.9) (end 190.1 123.9) (width 0.15) (layer "F.Cu") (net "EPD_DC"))
 (segment (start 118.9 141.4) (end 120 141.4) (width 0.15) (layer "F.Cu") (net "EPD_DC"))
 (segment (start 117.3 142.4) (end 118.9 141.4) (width 0.15) (layer "F.Cu") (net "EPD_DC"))
 (via (at 181.1 123.9) (size 0.5) (drill 0.3) (layers "F.Cu" "B.Cu") (capping no) (covering (front no) (back no))
  (plugging (front no) (back no)) (filling no) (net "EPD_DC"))
 (via (at 190.1 123.9) (size 0.5) (drill 0.3) (layers "F.Cu" "B.Cu") (capping no) (covering (front no) (back no))
  (plugging (front no) (back no)) (filling no) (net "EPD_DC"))
 (via (at 123.3 141.1) (size 0.5) (drill 0.3) (layers "F.Cu" "B.Cu") (capping no) (covering (front no) (back no))
  (plugging (front no) (back no)) (filling no) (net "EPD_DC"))
 (segment (start 155.9 123.9) (end 181.1 123.9) (width 0.15) (layer "B.Cu") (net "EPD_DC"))
 (segment (start 190.1 123.9) (end 191.7 123.9) (width 0.15) (layer "B.Cu") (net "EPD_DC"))
 (segment (start 123.3 141.1) (end 155.9 123.9) (width 0.15) (layer "B.Cu") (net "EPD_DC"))
 (segment (start 180.6 123.5) (end 186.8 118.8) (width 0.15) (layer "F.Cu") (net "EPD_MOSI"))
 (segment (start 179.3 125.7) (end 180.6 123.5) (width 0.15) (layer "F.Cu") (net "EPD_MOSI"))
 (segment (start 186.8 118.8) (end 189.5 118.8) (width 0.15) (layer "F.Cu") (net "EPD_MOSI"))
 (via (at 189.5 118.8) (size 0.5) (drill 0.3) (layers "F.Cu" "B.Cu") (capping no) (covering (front no) (back no))
  (plugging (front no) (back no)) (filling no) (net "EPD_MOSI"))
 (via (at 179.3 125.7) (size 0.5) (drill 0.3) (layers "F.Cu" "B.Cu") (capping no) (covering (front no) (back no))
  (plugging (front no) (back no)) (filling no) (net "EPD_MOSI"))
 (segment (start 130.4 142) (end 130.5 142.1) (width 0.15) (layer "B.Cu") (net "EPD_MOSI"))
 (segment (start 112.2 157.5) (end 130.4 142) (width 0.15) (layer "B.Cu") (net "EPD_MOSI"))
 (segment (start 130.5 142.1) (end 131.5 142.1) (width 0.15) (layer "B.Cu") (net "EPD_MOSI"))
 (segment (start 131.5 142.1) (end 179.3 125.7) (width 0.15) (layer "B.Cu") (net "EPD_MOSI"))
 (segment (start 189.5 118.8) (end 191.7 118.8) (width 0.15) (layer "B.Cu") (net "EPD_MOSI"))
 (segment (start 119.8 142.3) (end 129.699999 140.5) (width 0.15) (layer "F.Cu") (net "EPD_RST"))
 (via (at 129.699999 140.5) (size 0.5) (drill 0.3) (layers "F.Cu" "B.Cu") (capping no) (covering (front no) (back no))
  (plugging (front no) (back no)) (filling no) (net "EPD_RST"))
 (segment (start 130.6 139.6) (end 131.3 139.6) (width 0.15) (layer "B.Cu") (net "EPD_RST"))
 (segment (start 129.699999 140.5) (end 130.6 139.6) (width 0.15) (layer "B.Cu") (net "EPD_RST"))
 (segment (start 131.3 139.6) (end 191.7 121.3) (width 0.15) (layer "B.Cu") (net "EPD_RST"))
 (segment (start 187.8 123.1) (end 190.5 118.2) (width 0.15) (layer "F.Cu") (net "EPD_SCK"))
 (via (at 187.8 123.1) (size 0.5) (drill 0.3) (layers "F.Cu" "B.Cu") (capping no) (covering (front no) (back no))
  (plugging (front no) (back no)) (filling no) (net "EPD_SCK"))
 (via (at 190.5 118.2) (size 0.5) (drill 0.3) (layers "F.Cu" "B.Cu") (capping no) (covering (front no) (back no))
  (plugging (front no) (back no)) (filling no) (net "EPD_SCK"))
 (segment (start 163.5 147.4) (end 187.8 123.1) (width 0.15) (layer "B.Cu") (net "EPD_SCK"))
 (segment (start 163.3 147.5) (end 163.5 147.4) (width 0.15) (layer "B.Cu") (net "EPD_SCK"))
 (segment (start 132 146.9) (end 134.199999 147.5) (width 0.15) (layer "B.Cu") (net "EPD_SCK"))
 (segment (start 190.5 118.2) (end 192 116.7) (width 0.15) (layer "B.Cu") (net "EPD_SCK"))
 (segment (start 134.199999 147.5) (end 163.3 147.5) (width 0.15) (layer "B.Cu") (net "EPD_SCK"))
 (segment (start 117.3 157.6) (end 132 146.9) (width 0.15) (layer "B.Cu") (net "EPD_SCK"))
 (segment (start 134.75 152.354) (end 134.75 150.75) (width 0.15) (layer "F.Cu") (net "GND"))
 (segment (start 149.448 126.212775) (end 164.500775 111.16) (width 0.15) (layer "F.Cu") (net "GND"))
 (segment (start 109.2515 155.052) (end 132.052 155.052) (width 0.15) (layer "F.Cu") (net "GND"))
 (segment (start 160.860001 148.860001) (end 160.860001 142.399999) (width 0.15) (layer "F.Cu") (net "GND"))
 (segment (start 160.860001 142.399999) (end 161.66 141.6) (width 0.15) (layer "F.Cu") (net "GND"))
 (segment (start 164.500775 111.16) (end 192.5 111.16) (width 0.15) (layer "F.Cu") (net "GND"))
 (segment (start 149.448 126.587225) (end 149.448 126.212775) (width 0.15) (layer "F.Cu") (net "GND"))
 (segment (start 132.052 155.052) (end 134.75 152.354) (width 0.15) (layer "F.Cu") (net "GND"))
 (segment (start 167.5 141.6) (end 152.752 126.852) (width 0.15) (layer "F.Cu") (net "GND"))
 (segment (start 162.75 150.75) (end 160.860001 148.860001) (width 0.15) (layer "F.Cu") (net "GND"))
 (segment (start 106.4835 157.82) (end 109.2515 155.052) (width 0.15) (layer "F.Cu") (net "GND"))
 (segment (start 152.752 126.852) (end 149.712775 126.852) (width 0.15) (layer "F.Cu") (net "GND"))
 (segment (start 149.712775 126.852) (end 149.448 126.587225) (width 0.15) (layer "F.Cu") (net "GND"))
 (segment (start 167.5 141.6) (end 166.498 142.602) (width 0.15) (layer "B.Cu") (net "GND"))
 (segment (start 166.498 142.602) (end 162.662 142.602) (width 0.15) (layer "B.Cu") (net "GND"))
 (segment (start 134.75 150.75) (end 169.25 150.75) (width 0.15) (layer "B.Cu") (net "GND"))
 (segment (start 162.662 142.602) (end 161.66 141.6) (width 0.15) (layer "B.Cu") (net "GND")))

